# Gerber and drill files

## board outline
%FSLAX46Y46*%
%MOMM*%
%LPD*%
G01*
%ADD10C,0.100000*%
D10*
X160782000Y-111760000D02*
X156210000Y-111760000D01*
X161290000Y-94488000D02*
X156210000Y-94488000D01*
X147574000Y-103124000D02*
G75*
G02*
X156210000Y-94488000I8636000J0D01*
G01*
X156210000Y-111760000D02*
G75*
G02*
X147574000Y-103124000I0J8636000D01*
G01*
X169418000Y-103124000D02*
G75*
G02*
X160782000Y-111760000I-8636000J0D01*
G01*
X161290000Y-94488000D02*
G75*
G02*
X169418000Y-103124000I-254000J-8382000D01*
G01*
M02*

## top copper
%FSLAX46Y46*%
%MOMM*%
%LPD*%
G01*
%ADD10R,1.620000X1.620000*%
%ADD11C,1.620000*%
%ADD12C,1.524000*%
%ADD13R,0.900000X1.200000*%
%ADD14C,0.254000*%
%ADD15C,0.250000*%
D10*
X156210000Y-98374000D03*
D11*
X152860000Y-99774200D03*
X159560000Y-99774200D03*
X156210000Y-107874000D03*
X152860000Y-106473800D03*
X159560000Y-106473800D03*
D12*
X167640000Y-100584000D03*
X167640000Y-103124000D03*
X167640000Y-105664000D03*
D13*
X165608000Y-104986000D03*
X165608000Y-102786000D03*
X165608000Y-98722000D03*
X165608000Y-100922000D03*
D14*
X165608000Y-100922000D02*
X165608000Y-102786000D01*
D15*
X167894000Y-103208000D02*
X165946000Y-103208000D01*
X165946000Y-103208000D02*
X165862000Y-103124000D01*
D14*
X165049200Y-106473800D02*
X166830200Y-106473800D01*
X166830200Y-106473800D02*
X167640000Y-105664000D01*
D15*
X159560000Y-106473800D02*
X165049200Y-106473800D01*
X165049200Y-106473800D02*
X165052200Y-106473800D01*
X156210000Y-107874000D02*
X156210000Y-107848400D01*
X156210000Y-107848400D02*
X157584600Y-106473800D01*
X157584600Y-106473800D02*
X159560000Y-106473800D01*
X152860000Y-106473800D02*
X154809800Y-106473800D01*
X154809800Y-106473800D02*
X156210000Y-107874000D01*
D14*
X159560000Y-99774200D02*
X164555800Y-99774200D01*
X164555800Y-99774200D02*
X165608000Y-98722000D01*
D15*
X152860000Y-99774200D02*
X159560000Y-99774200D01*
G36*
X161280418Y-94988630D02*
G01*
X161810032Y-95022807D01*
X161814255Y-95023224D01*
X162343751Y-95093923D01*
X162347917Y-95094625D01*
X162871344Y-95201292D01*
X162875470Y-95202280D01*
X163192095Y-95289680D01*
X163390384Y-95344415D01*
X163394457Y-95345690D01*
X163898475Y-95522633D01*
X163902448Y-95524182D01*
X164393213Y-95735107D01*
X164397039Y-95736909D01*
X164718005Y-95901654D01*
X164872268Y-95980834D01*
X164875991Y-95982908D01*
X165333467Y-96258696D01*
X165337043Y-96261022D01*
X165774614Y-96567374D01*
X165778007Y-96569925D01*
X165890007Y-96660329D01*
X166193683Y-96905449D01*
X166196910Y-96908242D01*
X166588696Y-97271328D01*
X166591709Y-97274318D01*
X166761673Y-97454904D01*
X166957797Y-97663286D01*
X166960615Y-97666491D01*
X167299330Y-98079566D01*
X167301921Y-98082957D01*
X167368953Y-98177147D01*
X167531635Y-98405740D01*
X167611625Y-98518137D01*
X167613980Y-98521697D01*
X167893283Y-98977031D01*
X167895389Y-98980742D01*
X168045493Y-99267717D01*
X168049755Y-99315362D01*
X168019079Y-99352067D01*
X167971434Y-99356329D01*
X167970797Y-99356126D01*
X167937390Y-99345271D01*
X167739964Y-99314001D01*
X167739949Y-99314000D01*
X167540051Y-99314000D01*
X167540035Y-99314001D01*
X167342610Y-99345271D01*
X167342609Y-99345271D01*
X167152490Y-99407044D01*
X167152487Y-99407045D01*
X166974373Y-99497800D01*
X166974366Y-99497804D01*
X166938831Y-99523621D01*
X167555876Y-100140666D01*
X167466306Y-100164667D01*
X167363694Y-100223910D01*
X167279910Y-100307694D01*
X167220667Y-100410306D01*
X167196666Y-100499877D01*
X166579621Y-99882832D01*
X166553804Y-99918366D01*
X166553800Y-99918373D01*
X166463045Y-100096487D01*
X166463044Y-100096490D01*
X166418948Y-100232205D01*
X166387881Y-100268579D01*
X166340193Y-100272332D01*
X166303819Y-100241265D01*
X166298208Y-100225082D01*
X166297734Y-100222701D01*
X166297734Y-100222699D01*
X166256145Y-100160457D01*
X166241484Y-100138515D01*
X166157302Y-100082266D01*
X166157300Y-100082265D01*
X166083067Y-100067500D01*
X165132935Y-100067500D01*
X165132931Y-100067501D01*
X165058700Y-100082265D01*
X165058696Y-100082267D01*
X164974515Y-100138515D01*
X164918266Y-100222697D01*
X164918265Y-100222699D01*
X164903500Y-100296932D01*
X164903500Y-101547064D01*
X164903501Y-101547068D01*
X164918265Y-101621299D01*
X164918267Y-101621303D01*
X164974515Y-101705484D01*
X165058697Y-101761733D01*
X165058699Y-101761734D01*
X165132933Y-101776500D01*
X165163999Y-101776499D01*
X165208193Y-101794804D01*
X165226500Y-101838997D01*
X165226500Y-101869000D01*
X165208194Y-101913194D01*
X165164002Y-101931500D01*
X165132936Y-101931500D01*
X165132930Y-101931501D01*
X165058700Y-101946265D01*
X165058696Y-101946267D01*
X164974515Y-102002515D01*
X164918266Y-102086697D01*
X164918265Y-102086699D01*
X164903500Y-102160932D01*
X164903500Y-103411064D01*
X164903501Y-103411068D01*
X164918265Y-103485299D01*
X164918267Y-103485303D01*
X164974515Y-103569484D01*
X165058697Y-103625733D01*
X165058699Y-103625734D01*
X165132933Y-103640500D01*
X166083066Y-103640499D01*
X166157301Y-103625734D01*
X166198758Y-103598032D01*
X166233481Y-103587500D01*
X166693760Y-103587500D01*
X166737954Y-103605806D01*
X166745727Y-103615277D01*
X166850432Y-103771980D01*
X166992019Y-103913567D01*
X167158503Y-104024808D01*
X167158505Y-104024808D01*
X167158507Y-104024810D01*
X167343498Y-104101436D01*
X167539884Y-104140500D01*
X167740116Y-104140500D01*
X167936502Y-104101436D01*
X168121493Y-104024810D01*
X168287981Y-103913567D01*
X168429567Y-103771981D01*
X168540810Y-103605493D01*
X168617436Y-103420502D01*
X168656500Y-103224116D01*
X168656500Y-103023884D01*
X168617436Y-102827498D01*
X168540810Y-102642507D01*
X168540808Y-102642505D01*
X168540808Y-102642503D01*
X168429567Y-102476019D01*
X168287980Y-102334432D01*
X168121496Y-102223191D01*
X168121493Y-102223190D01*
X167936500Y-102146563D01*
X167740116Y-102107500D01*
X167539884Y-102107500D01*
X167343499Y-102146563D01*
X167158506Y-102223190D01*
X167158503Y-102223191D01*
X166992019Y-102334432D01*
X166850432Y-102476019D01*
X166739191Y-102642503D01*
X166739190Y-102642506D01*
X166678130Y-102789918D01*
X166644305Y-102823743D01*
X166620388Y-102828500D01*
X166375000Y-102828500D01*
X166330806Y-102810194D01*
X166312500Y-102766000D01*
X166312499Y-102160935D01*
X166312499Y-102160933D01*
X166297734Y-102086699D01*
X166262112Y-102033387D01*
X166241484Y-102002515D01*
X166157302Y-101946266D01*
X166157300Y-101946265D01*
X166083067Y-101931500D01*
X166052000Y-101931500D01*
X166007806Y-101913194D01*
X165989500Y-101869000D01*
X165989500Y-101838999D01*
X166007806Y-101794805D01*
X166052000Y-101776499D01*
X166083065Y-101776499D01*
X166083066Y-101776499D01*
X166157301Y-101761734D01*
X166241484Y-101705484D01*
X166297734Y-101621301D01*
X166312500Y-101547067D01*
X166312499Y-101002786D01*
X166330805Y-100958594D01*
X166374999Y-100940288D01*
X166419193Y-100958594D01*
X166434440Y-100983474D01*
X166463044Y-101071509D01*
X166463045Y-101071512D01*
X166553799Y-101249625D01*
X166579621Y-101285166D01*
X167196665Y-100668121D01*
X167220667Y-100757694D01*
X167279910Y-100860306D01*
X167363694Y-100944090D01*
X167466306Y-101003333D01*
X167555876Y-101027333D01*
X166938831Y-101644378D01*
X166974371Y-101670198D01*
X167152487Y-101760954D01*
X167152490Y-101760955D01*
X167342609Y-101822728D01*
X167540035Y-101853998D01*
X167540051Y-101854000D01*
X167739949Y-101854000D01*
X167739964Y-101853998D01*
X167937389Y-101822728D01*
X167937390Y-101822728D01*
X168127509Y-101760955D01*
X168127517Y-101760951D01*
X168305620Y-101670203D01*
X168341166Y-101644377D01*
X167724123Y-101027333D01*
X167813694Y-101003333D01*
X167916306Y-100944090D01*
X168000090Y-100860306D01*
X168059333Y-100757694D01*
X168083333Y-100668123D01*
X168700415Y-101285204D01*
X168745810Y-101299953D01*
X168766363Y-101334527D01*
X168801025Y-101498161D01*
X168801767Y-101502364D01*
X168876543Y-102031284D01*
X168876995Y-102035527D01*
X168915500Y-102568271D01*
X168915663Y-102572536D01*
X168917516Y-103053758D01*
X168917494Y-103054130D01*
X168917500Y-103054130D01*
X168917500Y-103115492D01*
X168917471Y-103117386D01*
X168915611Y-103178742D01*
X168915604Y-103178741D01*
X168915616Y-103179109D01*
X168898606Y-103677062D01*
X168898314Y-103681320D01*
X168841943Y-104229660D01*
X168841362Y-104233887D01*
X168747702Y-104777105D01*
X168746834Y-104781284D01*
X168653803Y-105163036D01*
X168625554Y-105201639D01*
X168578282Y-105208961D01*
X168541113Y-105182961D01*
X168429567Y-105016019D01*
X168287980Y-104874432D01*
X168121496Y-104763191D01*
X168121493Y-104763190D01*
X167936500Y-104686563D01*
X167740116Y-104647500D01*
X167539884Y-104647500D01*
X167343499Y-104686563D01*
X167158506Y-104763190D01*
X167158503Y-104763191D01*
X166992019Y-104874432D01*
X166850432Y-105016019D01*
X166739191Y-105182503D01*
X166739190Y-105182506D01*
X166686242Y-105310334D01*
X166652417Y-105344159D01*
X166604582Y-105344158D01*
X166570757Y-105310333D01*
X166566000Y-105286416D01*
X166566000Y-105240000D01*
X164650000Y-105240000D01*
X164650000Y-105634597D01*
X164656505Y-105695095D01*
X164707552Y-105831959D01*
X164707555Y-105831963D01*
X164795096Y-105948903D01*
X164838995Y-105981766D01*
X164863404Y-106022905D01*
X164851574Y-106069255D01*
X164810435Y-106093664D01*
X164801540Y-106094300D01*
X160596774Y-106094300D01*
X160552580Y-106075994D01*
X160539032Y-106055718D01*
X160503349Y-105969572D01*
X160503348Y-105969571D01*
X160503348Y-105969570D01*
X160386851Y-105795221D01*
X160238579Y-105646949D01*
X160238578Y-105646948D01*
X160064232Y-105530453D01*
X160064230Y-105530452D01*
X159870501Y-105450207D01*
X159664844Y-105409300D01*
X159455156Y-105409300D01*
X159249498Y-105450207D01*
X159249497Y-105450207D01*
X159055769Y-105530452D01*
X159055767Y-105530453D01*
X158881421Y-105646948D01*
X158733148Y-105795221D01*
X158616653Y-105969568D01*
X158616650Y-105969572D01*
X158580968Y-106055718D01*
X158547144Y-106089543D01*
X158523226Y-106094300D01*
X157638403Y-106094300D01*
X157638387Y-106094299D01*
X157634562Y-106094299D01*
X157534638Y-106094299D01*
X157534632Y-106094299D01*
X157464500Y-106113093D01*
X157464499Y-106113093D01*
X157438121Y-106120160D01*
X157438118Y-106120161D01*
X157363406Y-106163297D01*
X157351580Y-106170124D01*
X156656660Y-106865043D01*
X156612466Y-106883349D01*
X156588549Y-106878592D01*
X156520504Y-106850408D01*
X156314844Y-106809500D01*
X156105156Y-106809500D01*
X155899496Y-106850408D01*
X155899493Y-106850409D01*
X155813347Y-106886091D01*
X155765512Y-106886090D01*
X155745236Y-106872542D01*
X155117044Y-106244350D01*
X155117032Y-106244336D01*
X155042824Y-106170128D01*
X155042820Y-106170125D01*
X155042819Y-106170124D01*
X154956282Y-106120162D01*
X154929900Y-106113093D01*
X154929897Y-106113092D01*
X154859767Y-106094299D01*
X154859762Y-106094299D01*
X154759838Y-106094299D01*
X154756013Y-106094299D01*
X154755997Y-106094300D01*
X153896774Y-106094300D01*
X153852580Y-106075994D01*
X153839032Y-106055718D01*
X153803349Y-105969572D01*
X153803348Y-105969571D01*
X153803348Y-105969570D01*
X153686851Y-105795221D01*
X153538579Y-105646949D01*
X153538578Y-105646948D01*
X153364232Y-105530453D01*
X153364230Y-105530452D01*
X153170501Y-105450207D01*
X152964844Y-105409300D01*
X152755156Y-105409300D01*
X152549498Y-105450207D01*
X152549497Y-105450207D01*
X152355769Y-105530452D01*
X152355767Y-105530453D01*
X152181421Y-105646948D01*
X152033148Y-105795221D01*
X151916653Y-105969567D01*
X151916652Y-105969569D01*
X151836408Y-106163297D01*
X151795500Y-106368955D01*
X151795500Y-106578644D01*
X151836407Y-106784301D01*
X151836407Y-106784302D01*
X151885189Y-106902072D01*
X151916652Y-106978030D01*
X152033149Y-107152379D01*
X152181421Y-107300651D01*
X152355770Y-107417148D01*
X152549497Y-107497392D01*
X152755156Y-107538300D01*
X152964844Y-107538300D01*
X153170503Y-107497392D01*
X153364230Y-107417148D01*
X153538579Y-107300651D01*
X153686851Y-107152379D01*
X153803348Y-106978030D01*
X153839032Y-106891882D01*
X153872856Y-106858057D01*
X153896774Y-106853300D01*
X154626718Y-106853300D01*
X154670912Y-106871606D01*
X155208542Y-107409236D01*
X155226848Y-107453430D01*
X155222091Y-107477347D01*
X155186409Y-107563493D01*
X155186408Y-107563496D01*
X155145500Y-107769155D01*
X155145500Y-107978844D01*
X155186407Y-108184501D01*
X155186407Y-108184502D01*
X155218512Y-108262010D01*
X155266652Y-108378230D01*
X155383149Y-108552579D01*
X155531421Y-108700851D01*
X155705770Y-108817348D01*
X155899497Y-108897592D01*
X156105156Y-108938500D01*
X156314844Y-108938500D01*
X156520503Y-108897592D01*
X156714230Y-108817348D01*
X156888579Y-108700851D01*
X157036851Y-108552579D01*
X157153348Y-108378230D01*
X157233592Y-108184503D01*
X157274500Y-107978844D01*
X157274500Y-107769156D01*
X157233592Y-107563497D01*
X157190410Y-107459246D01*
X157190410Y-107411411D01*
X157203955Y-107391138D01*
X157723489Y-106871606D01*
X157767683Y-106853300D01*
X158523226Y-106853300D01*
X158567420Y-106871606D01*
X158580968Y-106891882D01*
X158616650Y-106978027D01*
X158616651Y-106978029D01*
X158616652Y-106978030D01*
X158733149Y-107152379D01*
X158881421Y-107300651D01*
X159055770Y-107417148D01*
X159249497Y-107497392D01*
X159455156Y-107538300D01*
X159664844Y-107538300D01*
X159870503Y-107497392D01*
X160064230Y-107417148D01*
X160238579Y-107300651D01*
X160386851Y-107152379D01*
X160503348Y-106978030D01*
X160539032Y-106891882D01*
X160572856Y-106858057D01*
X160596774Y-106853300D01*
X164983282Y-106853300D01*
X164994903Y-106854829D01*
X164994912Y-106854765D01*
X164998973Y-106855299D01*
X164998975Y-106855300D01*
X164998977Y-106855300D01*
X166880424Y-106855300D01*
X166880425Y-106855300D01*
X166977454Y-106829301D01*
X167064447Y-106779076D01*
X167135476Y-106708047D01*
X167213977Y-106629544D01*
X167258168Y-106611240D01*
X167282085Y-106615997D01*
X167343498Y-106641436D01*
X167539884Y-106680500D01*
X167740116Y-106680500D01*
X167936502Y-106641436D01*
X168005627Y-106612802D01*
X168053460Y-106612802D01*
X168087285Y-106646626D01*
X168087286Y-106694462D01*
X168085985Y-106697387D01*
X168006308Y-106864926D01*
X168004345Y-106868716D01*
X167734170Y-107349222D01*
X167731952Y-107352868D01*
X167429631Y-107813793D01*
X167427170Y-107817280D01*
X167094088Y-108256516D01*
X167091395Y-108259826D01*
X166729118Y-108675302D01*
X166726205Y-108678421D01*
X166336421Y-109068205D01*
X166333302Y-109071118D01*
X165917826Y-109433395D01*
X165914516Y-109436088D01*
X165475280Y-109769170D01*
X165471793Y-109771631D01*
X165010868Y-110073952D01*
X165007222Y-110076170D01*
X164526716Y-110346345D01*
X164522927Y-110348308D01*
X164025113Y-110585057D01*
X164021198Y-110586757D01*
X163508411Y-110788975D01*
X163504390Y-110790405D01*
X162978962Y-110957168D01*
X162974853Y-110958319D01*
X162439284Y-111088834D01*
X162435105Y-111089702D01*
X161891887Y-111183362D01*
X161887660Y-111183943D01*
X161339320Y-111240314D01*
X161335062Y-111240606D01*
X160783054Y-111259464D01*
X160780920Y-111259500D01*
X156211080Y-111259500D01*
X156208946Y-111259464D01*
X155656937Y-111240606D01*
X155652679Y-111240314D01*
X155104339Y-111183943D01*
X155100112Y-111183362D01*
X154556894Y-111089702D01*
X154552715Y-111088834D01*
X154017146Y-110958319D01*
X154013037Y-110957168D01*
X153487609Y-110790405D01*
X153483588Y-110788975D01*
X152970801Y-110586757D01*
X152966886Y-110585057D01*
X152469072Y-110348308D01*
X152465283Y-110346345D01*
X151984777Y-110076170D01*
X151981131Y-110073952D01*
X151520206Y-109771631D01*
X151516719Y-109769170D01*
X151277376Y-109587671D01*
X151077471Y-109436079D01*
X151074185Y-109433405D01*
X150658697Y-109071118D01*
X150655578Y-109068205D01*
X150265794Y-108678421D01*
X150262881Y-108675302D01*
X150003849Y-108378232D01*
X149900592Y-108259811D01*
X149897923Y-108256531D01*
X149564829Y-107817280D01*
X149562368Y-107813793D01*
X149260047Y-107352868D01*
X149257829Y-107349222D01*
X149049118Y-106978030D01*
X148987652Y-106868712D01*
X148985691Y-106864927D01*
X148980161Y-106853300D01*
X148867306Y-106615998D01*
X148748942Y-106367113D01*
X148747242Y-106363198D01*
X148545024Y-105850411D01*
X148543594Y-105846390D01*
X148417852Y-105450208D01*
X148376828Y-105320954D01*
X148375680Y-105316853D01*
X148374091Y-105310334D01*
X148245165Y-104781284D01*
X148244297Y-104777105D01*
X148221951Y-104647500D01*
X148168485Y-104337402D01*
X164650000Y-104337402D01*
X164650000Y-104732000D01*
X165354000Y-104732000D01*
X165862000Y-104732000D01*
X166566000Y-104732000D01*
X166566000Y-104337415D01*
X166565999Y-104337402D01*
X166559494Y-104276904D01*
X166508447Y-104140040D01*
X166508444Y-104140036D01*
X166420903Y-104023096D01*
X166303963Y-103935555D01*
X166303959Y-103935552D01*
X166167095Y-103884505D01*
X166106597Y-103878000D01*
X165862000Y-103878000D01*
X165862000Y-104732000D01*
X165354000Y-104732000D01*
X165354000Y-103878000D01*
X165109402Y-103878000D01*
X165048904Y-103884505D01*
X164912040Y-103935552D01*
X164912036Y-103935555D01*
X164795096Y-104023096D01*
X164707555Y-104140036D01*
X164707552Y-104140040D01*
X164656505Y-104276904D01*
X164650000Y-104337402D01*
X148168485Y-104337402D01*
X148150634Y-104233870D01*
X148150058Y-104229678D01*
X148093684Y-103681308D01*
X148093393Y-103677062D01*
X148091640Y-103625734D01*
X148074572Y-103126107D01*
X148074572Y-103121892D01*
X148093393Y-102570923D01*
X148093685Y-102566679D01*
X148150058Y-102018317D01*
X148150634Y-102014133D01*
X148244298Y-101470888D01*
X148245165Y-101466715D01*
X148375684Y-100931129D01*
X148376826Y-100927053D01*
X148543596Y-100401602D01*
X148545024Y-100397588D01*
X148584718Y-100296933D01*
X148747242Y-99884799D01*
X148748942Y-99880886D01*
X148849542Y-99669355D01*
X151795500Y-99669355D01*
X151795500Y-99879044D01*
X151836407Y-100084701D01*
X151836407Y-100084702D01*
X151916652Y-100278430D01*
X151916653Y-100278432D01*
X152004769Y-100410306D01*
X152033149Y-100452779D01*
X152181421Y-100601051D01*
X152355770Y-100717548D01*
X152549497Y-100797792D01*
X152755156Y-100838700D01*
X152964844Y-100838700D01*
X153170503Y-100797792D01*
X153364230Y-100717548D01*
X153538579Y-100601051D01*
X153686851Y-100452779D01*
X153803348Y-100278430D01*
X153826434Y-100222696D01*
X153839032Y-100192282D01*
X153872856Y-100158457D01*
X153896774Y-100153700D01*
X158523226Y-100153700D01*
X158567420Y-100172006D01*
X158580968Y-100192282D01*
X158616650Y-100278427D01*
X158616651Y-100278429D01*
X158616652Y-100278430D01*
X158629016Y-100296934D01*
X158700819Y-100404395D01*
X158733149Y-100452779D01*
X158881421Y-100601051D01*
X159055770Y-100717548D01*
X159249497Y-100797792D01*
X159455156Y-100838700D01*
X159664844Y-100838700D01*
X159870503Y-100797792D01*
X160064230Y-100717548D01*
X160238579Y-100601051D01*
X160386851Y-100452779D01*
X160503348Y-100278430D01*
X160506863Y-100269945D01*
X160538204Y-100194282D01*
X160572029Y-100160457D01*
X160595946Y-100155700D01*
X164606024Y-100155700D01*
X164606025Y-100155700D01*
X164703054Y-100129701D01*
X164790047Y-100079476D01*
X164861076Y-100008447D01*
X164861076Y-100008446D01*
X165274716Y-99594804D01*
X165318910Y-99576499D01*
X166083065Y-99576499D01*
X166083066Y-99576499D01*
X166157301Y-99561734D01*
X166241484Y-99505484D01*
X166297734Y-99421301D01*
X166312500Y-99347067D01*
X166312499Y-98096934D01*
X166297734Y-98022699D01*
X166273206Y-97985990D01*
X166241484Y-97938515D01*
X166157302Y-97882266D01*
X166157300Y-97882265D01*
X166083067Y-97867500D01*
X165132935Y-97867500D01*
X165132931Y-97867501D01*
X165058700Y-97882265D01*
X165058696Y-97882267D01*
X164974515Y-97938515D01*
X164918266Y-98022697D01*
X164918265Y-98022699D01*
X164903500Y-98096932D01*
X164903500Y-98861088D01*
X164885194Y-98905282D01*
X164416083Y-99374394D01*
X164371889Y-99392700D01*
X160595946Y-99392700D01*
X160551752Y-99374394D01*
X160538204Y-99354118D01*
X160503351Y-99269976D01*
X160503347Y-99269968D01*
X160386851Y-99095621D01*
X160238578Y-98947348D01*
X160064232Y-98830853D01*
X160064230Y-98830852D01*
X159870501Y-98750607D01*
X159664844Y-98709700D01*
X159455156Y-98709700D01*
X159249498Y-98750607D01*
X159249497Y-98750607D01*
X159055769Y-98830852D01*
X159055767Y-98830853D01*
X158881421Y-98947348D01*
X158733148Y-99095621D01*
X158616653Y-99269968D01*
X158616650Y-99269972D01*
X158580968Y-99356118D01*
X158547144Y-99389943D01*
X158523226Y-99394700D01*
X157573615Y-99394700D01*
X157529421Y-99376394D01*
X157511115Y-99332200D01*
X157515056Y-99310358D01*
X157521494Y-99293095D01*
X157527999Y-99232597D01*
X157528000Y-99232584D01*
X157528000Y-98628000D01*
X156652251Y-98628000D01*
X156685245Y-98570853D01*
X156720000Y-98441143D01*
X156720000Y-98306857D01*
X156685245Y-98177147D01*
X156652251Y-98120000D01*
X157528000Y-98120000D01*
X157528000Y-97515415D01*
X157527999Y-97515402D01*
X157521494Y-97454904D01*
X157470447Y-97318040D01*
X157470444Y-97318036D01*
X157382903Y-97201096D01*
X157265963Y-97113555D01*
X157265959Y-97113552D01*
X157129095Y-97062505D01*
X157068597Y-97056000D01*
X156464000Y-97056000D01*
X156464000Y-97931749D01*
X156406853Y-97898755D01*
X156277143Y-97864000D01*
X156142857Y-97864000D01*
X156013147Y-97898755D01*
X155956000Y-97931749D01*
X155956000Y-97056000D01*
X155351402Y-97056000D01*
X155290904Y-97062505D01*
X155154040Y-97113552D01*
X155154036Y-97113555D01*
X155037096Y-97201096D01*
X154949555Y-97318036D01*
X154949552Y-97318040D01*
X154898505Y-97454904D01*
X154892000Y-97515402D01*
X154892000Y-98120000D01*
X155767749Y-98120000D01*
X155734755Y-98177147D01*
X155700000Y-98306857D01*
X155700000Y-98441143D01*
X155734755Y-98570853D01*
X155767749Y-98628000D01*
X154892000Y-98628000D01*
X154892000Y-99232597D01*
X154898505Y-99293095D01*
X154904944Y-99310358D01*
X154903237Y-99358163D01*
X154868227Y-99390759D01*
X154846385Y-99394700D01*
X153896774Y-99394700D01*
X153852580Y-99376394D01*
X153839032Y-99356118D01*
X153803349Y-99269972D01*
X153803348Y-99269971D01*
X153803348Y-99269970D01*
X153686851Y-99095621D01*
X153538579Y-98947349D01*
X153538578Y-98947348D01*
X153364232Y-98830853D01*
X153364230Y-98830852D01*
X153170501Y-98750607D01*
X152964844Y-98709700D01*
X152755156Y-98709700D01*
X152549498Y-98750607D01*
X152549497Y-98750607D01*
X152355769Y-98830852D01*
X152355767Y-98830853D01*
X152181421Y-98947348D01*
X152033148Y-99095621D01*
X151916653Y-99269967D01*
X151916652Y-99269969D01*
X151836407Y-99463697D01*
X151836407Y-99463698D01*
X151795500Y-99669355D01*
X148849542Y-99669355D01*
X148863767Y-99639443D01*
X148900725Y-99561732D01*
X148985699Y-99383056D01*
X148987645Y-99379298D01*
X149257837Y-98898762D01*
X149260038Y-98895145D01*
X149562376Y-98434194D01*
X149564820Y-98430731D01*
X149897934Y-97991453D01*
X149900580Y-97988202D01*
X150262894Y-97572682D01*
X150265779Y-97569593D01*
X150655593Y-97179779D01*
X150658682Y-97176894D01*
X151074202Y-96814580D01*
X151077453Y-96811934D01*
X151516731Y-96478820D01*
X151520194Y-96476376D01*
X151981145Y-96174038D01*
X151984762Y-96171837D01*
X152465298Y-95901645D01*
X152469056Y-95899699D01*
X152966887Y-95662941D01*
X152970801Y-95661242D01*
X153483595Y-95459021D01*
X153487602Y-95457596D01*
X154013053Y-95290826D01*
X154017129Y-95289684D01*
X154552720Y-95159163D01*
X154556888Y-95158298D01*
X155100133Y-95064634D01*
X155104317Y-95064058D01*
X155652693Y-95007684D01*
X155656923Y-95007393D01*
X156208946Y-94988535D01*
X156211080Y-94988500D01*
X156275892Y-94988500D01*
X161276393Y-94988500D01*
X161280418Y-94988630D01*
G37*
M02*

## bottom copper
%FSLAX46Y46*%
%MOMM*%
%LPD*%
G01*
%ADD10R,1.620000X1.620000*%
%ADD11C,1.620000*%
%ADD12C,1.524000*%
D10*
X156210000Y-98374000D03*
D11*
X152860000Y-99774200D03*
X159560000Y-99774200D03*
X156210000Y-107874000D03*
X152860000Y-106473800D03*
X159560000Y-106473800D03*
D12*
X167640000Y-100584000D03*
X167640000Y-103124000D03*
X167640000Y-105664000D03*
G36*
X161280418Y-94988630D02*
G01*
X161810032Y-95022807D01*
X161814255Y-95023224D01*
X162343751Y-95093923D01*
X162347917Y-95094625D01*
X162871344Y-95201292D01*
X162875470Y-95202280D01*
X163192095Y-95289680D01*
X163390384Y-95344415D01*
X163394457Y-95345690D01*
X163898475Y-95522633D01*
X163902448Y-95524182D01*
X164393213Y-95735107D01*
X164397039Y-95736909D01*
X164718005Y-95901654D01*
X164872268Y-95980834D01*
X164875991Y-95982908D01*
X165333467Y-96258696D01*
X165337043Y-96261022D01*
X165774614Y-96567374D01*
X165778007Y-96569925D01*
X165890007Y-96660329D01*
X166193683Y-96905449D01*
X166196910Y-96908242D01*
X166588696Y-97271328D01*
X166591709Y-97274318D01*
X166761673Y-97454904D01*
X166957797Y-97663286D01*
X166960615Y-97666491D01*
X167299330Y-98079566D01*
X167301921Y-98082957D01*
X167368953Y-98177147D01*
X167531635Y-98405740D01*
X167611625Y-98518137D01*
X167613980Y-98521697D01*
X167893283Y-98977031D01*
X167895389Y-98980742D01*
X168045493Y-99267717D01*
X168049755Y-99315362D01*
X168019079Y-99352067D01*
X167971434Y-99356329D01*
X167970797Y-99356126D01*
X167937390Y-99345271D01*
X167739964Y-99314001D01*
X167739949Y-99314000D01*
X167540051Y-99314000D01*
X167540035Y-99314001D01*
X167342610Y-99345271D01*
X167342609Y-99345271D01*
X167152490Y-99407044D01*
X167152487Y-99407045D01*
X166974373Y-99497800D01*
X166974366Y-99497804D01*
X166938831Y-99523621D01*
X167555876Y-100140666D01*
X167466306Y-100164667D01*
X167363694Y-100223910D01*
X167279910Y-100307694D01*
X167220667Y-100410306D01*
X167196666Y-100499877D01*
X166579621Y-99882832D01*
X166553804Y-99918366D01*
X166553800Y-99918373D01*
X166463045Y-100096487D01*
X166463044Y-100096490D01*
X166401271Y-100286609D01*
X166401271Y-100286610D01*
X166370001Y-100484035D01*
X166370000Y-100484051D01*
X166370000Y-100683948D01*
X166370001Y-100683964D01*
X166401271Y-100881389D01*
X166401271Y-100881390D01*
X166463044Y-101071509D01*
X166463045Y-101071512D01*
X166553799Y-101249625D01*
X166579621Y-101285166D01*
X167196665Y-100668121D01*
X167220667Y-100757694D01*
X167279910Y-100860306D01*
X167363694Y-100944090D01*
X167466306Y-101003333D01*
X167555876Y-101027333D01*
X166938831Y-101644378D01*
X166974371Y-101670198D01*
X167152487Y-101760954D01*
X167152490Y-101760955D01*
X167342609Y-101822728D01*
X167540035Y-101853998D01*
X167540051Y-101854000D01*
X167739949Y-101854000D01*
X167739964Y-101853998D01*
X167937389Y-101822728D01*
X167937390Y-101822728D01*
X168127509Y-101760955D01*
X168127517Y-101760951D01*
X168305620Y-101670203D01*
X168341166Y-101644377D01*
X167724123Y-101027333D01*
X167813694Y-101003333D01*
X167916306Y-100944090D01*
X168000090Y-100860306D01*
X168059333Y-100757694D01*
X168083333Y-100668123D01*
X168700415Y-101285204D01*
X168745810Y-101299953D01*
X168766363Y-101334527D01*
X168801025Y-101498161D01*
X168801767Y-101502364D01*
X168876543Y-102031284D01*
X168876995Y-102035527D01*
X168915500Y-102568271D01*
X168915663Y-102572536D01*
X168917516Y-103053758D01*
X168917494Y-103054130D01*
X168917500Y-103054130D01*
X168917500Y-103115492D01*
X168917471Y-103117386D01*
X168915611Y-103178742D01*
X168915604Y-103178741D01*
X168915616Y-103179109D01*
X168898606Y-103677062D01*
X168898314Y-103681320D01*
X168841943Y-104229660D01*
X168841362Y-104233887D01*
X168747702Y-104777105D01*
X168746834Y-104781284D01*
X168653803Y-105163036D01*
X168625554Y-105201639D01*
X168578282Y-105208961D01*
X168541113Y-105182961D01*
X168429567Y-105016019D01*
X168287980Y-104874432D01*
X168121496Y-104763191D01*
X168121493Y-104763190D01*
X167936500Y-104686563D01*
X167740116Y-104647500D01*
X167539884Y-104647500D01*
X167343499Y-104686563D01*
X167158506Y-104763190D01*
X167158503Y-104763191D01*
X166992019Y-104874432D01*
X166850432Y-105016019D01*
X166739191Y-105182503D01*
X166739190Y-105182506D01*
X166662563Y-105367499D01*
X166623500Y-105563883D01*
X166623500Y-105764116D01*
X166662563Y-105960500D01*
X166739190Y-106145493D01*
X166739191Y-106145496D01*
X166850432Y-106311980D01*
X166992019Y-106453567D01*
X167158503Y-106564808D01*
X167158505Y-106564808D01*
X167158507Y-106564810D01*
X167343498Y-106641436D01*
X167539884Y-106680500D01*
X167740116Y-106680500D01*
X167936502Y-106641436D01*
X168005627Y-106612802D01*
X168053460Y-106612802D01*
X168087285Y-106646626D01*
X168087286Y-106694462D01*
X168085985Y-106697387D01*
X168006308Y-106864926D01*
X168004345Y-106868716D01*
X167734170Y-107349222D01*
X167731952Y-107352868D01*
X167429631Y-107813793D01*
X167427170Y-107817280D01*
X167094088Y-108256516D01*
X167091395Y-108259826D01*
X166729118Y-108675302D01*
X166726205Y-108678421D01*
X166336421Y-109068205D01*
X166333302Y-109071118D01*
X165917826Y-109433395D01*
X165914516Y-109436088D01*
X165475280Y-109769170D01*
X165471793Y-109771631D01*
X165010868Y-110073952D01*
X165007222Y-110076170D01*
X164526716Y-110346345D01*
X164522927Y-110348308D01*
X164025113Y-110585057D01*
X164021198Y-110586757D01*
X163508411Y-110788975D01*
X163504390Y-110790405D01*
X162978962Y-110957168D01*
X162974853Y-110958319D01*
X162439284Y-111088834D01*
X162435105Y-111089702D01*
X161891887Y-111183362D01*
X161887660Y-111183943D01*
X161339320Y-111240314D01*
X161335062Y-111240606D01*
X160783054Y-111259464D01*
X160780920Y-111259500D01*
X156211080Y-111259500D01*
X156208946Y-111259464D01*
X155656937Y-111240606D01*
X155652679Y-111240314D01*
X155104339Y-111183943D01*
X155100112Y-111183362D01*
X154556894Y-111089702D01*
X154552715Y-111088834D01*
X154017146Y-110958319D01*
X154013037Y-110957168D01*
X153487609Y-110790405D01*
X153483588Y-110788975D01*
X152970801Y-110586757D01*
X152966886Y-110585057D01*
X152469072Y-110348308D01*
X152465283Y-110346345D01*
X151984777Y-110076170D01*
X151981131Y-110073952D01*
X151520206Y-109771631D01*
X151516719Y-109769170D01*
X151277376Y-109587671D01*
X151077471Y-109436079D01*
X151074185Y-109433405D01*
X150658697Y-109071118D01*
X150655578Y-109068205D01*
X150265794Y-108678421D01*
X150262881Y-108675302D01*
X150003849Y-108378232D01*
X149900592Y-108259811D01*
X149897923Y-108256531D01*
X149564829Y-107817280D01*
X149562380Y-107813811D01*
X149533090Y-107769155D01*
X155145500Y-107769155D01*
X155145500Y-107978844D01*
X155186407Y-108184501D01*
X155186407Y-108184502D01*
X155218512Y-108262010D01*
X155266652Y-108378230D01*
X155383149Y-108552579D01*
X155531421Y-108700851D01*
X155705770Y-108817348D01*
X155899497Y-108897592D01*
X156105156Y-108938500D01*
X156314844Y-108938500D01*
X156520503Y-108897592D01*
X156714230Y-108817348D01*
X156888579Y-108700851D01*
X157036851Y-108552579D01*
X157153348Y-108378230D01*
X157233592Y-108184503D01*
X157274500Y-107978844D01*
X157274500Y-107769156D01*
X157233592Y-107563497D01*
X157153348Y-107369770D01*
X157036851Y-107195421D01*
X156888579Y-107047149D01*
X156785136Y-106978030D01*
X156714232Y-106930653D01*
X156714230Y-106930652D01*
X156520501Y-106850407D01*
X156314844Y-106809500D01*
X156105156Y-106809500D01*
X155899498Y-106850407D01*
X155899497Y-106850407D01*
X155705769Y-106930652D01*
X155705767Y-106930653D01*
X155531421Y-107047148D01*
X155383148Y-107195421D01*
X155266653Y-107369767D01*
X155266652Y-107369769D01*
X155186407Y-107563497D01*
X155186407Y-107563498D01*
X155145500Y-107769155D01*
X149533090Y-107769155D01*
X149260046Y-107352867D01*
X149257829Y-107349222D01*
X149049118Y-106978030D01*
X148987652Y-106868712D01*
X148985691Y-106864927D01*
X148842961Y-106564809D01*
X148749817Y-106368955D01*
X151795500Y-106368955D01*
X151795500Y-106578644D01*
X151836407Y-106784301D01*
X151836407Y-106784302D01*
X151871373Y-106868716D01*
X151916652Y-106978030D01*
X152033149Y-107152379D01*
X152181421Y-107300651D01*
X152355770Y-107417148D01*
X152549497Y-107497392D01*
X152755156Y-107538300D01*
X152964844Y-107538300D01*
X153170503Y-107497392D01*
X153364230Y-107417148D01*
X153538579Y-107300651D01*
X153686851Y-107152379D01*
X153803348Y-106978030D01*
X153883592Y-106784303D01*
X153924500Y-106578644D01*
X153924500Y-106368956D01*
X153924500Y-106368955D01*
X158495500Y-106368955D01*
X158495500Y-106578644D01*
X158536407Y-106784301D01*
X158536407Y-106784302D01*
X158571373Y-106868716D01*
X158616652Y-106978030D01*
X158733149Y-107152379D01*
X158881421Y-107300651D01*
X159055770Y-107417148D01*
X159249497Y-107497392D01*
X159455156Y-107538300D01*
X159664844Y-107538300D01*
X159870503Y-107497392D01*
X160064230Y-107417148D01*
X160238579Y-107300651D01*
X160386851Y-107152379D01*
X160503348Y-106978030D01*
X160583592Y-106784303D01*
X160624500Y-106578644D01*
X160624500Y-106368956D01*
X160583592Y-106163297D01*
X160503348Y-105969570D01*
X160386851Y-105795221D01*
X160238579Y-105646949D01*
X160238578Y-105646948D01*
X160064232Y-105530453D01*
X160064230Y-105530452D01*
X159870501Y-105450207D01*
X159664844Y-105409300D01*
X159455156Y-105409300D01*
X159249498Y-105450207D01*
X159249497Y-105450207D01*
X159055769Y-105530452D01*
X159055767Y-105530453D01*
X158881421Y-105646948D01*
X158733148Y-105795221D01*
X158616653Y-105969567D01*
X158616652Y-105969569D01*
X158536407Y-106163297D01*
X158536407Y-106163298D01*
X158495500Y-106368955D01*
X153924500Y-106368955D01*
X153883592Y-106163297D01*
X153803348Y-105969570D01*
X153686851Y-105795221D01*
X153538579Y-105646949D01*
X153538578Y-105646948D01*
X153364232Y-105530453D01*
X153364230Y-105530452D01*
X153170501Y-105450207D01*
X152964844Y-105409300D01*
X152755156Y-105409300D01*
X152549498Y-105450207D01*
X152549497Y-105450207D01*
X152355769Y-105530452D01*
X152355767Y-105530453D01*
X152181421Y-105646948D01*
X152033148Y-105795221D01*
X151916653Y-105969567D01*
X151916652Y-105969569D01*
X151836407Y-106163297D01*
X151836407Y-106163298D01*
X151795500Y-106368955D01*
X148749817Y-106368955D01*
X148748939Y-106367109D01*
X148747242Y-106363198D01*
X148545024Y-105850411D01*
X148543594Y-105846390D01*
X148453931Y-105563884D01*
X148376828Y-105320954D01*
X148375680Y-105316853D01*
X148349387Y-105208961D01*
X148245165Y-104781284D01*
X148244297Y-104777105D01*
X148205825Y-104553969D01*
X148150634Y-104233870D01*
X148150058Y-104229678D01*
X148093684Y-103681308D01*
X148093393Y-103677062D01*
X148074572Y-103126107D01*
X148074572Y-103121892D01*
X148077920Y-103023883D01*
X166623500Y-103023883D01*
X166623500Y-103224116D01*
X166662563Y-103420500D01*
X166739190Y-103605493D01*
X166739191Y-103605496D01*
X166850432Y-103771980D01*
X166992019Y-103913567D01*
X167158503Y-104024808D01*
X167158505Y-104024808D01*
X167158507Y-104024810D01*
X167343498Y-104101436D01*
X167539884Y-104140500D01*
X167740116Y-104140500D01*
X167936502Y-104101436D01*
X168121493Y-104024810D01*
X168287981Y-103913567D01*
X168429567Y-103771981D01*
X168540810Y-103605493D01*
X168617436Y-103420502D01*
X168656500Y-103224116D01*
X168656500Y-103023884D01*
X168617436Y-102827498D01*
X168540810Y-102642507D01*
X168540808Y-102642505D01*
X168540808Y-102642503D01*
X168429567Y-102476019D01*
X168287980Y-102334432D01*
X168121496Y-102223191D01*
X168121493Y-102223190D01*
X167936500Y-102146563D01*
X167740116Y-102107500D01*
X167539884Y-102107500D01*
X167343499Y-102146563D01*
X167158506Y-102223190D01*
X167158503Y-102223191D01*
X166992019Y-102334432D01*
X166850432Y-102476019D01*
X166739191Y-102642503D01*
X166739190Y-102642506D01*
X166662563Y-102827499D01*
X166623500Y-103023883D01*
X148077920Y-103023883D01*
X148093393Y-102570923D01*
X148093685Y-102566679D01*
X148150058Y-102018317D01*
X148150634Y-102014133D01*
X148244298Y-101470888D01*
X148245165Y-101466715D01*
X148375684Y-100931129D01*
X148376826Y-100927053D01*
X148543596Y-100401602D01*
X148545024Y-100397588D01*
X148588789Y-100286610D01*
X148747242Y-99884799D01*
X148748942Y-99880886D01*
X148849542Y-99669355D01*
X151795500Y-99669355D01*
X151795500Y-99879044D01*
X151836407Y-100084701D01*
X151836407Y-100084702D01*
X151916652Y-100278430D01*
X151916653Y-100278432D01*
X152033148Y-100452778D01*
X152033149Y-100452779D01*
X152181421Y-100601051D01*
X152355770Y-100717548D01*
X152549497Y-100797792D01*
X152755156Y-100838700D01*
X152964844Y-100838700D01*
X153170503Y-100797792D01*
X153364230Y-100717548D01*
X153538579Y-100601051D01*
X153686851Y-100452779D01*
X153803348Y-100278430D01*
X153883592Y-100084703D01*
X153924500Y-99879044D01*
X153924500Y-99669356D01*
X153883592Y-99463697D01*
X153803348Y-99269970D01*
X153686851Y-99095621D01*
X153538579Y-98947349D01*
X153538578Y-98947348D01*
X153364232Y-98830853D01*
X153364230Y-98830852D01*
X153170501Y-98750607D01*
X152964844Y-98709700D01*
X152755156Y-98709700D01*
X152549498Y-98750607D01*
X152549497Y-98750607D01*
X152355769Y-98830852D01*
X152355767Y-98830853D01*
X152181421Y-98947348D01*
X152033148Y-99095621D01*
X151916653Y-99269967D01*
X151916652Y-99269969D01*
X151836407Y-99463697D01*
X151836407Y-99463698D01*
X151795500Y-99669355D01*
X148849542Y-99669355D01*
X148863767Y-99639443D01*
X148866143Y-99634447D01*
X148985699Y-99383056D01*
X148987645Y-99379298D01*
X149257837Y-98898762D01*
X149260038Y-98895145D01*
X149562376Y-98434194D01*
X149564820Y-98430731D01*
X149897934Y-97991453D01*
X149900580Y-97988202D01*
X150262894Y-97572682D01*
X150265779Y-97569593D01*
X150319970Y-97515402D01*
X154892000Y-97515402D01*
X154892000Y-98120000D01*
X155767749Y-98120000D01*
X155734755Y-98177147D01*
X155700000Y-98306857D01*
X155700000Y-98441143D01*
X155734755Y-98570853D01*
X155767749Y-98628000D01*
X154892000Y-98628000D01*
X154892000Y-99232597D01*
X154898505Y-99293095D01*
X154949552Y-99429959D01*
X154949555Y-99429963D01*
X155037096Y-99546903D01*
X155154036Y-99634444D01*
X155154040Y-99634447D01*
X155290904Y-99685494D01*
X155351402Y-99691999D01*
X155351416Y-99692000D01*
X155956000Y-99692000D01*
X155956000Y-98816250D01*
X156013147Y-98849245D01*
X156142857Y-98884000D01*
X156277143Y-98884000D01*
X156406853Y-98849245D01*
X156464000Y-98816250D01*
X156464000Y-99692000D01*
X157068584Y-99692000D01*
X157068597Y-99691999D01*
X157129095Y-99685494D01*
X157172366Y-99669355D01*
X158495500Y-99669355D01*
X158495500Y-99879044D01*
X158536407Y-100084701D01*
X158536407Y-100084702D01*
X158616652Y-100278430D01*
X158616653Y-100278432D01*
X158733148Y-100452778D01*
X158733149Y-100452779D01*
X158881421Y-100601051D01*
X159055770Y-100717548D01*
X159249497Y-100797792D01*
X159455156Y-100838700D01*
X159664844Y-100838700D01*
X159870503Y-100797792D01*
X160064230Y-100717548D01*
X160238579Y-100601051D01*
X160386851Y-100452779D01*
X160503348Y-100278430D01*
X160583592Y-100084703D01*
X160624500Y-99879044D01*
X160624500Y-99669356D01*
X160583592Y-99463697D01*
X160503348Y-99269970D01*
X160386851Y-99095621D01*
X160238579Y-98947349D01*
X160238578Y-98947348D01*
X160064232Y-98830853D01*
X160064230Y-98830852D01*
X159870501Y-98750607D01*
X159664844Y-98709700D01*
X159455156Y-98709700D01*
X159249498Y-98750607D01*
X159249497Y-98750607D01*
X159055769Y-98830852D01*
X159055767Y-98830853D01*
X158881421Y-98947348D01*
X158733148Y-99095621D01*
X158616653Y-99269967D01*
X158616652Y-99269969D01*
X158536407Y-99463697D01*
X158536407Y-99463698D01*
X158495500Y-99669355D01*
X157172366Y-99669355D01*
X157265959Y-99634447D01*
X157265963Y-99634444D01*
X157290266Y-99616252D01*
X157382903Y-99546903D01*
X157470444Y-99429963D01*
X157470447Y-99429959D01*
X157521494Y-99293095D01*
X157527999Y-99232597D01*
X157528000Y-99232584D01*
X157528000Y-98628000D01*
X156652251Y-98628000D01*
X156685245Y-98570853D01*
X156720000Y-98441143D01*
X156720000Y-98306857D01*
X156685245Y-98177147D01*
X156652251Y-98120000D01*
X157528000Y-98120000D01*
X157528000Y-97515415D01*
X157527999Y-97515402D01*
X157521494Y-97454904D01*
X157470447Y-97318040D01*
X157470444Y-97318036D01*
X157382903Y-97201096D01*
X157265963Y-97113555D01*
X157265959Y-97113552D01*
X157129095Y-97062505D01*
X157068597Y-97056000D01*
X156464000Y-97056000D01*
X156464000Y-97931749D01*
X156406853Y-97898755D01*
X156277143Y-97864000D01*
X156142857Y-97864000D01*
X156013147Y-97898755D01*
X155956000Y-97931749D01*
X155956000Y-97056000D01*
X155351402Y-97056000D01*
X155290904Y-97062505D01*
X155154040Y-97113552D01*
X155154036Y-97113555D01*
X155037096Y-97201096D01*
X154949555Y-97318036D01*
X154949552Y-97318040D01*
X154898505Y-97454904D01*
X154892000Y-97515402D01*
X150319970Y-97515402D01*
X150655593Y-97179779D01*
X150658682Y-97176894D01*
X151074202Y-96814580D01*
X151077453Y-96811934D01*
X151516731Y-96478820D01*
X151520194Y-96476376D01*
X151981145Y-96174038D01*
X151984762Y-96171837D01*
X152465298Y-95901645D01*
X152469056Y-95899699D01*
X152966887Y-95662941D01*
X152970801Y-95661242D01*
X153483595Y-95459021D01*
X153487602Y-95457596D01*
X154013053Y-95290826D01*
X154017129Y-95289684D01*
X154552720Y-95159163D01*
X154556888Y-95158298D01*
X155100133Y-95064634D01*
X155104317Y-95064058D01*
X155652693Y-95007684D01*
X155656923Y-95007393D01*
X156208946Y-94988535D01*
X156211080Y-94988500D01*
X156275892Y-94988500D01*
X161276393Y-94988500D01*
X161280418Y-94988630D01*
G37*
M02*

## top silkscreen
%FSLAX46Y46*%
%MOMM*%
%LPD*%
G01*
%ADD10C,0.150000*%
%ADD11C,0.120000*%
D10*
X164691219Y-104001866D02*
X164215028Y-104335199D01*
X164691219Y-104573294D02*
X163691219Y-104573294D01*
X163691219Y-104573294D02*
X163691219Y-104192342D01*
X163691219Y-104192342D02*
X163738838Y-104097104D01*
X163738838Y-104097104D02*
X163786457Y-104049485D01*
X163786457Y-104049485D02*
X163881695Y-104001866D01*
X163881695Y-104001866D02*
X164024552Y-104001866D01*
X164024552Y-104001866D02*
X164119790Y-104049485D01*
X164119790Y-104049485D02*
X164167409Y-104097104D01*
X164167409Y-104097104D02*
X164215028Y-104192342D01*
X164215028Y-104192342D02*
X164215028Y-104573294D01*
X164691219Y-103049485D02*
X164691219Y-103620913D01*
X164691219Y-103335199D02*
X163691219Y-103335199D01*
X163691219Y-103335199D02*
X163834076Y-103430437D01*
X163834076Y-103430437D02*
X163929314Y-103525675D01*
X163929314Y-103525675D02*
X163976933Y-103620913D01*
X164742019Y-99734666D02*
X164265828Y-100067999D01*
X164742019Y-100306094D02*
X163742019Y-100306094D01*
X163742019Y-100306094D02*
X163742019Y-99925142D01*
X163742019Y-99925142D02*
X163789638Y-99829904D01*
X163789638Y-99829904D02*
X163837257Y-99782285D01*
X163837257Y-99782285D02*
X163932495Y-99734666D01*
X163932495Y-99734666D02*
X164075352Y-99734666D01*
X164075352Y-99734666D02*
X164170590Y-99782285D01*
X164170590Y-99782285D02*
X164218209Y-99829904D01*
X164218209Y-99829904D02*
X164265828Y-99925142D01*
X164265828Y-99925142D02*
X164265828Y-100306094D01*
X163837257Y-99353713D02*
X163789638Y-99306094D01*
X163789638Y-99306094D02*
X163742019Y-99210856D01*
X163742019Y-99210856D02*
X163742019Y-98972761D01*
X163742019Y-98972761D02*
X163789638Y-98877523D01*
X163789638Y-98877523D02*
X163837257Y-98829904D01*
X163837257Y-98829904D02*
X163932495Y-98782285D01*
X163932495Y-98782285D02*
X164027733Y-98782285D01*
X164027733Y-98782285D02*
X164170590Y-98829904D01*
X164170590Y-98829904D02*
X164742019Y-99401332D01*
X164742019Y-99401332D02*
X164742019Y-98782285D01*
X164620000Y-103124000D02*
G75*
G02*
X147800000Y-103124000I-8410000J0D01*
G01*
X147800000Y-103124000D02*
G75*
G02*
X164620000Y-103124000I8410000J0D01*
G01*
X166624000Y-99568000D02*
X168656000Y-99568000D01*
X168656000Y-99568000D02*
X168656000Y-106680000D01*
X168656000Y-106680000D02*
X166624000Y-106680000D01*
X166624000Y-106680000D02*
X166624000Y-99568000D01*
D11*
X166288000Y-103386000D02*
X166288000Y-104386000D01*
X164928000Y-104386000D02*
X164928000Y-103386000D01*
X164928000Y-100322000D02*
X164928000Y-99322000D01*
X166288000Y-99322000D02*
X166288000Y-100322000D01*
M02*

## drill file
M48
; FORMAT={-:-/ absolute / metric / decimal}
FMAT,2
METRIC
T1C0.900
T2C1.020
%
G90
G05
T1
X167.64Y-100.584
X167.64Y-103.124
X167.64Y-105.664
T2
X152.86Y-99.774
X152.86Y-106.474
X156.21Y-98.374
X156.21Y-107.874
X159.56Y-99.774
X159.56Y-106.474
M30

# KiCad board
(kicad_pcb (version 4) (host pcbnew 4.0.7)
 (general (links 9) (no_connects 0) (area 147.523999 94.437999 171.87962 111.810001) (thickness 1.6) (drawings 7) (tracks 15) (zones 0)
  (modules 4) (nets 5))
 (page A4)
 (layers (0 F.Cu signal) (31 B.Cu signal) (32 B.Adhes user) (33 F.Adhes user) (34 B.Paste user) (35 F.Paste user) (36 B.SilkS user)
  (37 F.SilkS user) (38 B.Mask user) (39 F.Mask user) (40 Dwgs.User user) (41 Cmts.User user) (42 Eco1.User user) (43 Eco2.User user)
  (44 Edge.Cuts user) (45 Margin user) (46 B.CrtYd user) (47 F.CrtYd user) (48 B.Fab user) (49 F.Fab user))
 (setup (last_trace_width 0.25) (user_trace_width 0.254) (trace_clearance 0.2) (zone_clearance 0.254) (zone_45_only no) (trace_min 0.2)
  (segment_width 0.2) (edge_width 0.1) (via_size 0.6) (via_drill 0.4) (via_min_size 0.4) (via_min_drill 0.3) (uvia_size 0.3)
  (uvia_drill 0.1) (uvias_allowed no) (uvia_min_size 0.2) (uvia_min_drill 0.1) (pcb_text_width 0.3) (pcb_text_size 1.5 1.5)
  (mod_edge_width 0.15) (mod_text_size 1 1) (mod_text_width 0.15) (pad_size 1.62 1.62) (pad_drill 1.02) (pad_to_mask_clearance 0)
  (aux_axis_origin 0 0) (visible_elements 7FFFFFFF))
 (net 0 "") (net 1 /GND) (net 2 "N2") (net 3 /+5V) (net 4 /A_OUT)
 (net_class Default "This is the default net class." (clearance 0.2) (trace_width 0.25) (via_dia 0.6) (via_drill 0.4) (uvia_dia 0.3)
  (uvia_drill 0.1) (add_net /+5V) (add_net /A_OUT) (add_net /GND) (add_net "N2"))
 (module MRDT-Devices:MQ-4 (layer F.Cu) (at 156.21 103.124 90)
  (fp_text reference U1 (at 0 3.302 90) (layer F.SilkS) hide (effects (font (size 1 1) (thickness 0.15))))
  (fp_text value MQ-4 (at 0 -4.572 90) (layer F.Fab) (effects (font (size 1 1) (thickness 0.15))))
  (fp_circle (center 0 0) (end 8.41 0) (layer F.SilkS) (width 0.15))
  (pad 3 thru_hole rect (at 4.75 0 90) (size 1.62 1.62) (drill 1.02) (layers *.Cu *.Mask) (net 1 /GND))
  (pad 2 thru_hole circle (at 3.3498 -3.35 90) (size 1.62 1.62) (drill 1.02) (layers *.Cu *.Mask) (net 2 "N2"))
  (pad 2 thru_hole circle (at 3.3498 3.35 90) (size 1.62 1.62) (drill 1.02) (layers *.Cu *.Mask) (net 2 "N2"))
  (pad 1 thru_hole circle (at -4.75 0 90) (size 1.62 1.62) (drill 1.02) (layers *.Cu *.Mask) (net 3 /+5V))
  (pad 1 thru_hole circle (at -3.3498 -3.35 90) (size 1.62 1.62) (drill 1.02) (layers *.Cu *.Mask) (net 3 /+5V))
  (pad 1 thru_hole circle (at -3.3498 3.35 90) (size 1.62 1.62) (drill 1.02) (layers *.Cu *.Mask) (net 3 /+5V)))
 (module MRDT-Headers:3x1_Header (layer F.Cu) (at 167.132 104.14)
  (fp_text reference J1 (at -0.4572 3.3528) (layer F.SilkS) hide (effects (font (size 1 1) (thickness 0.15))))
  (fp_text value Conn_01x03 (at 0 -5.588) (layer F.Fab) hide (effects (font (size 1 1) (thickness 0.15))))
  (fp_line (start -0.508 -4.572) (end 1.524 -4.572) (layer F.SilkS) (width 0.15))
  (fp_line (start 1.524 -4.572) (end 1.524 2.54) (layer F.SilkS) (width 0.15))
  (fp_line (start 1.524 2.54) (end -0.508 2.54) (layer F.SilkS) (width 0.15))
  (fp_line (start -0.508 2.54) (end -0.508 -4.572) (layer F.SilkS) (width 0.15))
  (pad 1 thru_hole circle (at 0.508 -3.556) (size 1.524 1.524) (drill 0.9) (layers *.Cu *.Mask) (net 1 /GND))
  (pad 2 thru_hole circle (at 0.508 -1.016) (size 1.524 1.524) (drill 0.9) (layers *.Cu *.Mask) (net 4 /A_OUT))
  (pad 3 thru_hole circle (at 0.508 1.524) (size 1.524 1.524) (drill 0.9) (layers *.Cu *.Mask) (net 3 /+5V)))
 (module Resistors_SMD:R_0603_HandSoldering (layer F.Cu) (at 165.608 103.886 90)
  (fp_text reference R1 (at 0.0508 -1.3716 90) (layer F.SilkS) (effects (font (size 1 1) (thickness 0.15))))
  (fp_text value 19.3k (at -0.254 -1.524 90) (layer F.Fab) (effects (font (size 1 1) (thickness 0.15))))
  (fp_line (start 0.5 0.68) (end -0.5 0.68) (layer F.SilkS) (width 0.12))
  (fp_line (start -0.5 -0.68) (end 0.5 -0.68) (layer F.SilkS) (width 0.12))
  (pad 1 smd rect (at -1.1 0 90) (size 1.2 0.9) (layers F.Cu F.Paste F.Mask) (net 1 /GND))
  (pad 2 smd rect (at 1.1 0 90) (size 1.2 0.9) (layers F.Cu F.Paste F.Mask) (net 4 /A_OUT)))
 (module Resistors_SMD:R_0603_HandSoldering (layer F.Cu) (at 165.608 99.822 270)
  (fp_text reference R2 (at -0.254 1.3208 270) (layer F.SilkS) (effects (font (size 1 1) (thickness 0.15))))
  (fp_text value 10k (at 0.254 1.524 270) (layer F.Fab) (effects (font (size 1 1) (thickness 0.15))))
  (fp_line (start 0.5 0.68) (end -0.5 0.68) (layer F.SilkS) (width 0.12))
  (fp_line (start -0.5 -0.68) (end 0.5 -0.68) (layer F.SilkS) (width 0.12))
  (pad 1 smd rect (at -1.1 0 270) (size 1.2 0.9) (layers F.Cu F.Paste F.Mask) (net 2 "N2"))
  (pad 2 smd rect (at 1.1 0 270) (size 1.2 0.9) (layers F.Cu F.Paste F.Mask) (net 4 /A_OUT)))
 (gr_line (start 160.782 111.76) (end 156.21 111.76) (angle 90) (layer Edge.Cuts) (width 0.1))
 (gr_line (start 161.29 94.488) (end 156.21 94.488) (angle 90) (layer Edge.Cuts) (width 0.1))
 (gr_arc (start 156.21 103.124) (end 147.574 103.124) (angle 90) (layer Edge.Cuts) (width 0.1))
 (gr_arc (start 156.21 103.124) (end 156.21 111.76) (angle 90) (layer Edge.Cuts) (width 0.1))
 (gr_arc (start 160.782 103.124) (end 169.418 103.124) (angle 90) (layer Edge.Cuts) (width 0.1))
 (gr_arc (start 161.036 102.87) (end 161.29 94.488) (angle 90) (layer Edge.Cuts) (width 0.1))
 (segment (start 165.608 100.922) (end 165.608 102.786) (width 0.254) (layer F.Cu) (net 4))
 (segment (start 167.894 103.208) (end 165.946 103.208) (width 0.25) (layer F.Cu) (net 4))
 (segment (start 165.946 103.208) (end 165.862 103.124) (width 0.25) (layer F.Cu) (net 4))
 (segment (start 165.0492 106.4738) (end 166.8302 106.4738) (width 0.254) (layer F.Cu) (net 3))
 (segment (start 166.8302 106.4738) (end 167.64 105.664) (width 0.254) (layer F.Cu) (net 3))
 (segment (start 159.56 106.4738) (end 165.0492 106.4738) (width 0.25) (layer F.Cu) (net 3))
 (segment (start 165.0492 106.4738) (end 165.0522 106.4738) (width 0.25) (layer F.Cu) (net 3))
 (segment (start 156.21 107.874) (end 156.21 107.8484) (width 0.25) (layer F.Cu) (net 3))
 (segment (start 156.21 107.8484) (end 157.5846 106.4738) (width 0.25) (layer F.Cu) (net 3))
 (segment (start 157.5846 106.4738) (end 159.56 106.4738) (width 0.25) (layer F.Cu) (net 3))
 (segment (start 152.86 106.4738) (end 154.8098 106.4738) (width 0.25) (layer F.Cu) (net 3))
 (segment (start 154.8098 106.4738) (end 156.21 107.874) (width 0.25) (layer F.Cu) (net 3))
 (segment (start 159.56 99.7742) (end 164.5558 99.7742) (width 0.254) (layer F.Cu) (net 2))
 (segment (start 164.5558 99.7742) (end 165.608 98.722) (width 0.254) (layer F.Cu) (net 2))
 (segment (start 152.86 99.7742) (end 159.56 99.7742) (width 0.25) (layer F.Cu) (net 2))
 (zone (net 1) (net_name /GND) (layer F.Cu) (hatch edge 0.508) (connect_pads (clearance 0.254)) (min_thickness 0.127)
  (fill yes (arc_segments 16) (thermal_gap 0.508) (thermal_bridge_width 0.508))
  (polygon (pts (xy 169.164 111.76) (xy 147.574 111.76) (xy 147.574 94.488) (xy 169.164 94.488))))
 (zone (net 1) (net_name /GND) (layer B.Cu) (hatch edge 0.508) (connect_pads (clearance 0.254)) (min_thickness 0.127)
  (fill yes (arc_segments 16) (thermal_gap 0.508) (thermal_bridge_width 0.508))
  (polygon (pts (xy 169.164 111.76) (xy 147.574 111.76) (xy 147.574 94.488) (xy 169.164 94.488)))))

